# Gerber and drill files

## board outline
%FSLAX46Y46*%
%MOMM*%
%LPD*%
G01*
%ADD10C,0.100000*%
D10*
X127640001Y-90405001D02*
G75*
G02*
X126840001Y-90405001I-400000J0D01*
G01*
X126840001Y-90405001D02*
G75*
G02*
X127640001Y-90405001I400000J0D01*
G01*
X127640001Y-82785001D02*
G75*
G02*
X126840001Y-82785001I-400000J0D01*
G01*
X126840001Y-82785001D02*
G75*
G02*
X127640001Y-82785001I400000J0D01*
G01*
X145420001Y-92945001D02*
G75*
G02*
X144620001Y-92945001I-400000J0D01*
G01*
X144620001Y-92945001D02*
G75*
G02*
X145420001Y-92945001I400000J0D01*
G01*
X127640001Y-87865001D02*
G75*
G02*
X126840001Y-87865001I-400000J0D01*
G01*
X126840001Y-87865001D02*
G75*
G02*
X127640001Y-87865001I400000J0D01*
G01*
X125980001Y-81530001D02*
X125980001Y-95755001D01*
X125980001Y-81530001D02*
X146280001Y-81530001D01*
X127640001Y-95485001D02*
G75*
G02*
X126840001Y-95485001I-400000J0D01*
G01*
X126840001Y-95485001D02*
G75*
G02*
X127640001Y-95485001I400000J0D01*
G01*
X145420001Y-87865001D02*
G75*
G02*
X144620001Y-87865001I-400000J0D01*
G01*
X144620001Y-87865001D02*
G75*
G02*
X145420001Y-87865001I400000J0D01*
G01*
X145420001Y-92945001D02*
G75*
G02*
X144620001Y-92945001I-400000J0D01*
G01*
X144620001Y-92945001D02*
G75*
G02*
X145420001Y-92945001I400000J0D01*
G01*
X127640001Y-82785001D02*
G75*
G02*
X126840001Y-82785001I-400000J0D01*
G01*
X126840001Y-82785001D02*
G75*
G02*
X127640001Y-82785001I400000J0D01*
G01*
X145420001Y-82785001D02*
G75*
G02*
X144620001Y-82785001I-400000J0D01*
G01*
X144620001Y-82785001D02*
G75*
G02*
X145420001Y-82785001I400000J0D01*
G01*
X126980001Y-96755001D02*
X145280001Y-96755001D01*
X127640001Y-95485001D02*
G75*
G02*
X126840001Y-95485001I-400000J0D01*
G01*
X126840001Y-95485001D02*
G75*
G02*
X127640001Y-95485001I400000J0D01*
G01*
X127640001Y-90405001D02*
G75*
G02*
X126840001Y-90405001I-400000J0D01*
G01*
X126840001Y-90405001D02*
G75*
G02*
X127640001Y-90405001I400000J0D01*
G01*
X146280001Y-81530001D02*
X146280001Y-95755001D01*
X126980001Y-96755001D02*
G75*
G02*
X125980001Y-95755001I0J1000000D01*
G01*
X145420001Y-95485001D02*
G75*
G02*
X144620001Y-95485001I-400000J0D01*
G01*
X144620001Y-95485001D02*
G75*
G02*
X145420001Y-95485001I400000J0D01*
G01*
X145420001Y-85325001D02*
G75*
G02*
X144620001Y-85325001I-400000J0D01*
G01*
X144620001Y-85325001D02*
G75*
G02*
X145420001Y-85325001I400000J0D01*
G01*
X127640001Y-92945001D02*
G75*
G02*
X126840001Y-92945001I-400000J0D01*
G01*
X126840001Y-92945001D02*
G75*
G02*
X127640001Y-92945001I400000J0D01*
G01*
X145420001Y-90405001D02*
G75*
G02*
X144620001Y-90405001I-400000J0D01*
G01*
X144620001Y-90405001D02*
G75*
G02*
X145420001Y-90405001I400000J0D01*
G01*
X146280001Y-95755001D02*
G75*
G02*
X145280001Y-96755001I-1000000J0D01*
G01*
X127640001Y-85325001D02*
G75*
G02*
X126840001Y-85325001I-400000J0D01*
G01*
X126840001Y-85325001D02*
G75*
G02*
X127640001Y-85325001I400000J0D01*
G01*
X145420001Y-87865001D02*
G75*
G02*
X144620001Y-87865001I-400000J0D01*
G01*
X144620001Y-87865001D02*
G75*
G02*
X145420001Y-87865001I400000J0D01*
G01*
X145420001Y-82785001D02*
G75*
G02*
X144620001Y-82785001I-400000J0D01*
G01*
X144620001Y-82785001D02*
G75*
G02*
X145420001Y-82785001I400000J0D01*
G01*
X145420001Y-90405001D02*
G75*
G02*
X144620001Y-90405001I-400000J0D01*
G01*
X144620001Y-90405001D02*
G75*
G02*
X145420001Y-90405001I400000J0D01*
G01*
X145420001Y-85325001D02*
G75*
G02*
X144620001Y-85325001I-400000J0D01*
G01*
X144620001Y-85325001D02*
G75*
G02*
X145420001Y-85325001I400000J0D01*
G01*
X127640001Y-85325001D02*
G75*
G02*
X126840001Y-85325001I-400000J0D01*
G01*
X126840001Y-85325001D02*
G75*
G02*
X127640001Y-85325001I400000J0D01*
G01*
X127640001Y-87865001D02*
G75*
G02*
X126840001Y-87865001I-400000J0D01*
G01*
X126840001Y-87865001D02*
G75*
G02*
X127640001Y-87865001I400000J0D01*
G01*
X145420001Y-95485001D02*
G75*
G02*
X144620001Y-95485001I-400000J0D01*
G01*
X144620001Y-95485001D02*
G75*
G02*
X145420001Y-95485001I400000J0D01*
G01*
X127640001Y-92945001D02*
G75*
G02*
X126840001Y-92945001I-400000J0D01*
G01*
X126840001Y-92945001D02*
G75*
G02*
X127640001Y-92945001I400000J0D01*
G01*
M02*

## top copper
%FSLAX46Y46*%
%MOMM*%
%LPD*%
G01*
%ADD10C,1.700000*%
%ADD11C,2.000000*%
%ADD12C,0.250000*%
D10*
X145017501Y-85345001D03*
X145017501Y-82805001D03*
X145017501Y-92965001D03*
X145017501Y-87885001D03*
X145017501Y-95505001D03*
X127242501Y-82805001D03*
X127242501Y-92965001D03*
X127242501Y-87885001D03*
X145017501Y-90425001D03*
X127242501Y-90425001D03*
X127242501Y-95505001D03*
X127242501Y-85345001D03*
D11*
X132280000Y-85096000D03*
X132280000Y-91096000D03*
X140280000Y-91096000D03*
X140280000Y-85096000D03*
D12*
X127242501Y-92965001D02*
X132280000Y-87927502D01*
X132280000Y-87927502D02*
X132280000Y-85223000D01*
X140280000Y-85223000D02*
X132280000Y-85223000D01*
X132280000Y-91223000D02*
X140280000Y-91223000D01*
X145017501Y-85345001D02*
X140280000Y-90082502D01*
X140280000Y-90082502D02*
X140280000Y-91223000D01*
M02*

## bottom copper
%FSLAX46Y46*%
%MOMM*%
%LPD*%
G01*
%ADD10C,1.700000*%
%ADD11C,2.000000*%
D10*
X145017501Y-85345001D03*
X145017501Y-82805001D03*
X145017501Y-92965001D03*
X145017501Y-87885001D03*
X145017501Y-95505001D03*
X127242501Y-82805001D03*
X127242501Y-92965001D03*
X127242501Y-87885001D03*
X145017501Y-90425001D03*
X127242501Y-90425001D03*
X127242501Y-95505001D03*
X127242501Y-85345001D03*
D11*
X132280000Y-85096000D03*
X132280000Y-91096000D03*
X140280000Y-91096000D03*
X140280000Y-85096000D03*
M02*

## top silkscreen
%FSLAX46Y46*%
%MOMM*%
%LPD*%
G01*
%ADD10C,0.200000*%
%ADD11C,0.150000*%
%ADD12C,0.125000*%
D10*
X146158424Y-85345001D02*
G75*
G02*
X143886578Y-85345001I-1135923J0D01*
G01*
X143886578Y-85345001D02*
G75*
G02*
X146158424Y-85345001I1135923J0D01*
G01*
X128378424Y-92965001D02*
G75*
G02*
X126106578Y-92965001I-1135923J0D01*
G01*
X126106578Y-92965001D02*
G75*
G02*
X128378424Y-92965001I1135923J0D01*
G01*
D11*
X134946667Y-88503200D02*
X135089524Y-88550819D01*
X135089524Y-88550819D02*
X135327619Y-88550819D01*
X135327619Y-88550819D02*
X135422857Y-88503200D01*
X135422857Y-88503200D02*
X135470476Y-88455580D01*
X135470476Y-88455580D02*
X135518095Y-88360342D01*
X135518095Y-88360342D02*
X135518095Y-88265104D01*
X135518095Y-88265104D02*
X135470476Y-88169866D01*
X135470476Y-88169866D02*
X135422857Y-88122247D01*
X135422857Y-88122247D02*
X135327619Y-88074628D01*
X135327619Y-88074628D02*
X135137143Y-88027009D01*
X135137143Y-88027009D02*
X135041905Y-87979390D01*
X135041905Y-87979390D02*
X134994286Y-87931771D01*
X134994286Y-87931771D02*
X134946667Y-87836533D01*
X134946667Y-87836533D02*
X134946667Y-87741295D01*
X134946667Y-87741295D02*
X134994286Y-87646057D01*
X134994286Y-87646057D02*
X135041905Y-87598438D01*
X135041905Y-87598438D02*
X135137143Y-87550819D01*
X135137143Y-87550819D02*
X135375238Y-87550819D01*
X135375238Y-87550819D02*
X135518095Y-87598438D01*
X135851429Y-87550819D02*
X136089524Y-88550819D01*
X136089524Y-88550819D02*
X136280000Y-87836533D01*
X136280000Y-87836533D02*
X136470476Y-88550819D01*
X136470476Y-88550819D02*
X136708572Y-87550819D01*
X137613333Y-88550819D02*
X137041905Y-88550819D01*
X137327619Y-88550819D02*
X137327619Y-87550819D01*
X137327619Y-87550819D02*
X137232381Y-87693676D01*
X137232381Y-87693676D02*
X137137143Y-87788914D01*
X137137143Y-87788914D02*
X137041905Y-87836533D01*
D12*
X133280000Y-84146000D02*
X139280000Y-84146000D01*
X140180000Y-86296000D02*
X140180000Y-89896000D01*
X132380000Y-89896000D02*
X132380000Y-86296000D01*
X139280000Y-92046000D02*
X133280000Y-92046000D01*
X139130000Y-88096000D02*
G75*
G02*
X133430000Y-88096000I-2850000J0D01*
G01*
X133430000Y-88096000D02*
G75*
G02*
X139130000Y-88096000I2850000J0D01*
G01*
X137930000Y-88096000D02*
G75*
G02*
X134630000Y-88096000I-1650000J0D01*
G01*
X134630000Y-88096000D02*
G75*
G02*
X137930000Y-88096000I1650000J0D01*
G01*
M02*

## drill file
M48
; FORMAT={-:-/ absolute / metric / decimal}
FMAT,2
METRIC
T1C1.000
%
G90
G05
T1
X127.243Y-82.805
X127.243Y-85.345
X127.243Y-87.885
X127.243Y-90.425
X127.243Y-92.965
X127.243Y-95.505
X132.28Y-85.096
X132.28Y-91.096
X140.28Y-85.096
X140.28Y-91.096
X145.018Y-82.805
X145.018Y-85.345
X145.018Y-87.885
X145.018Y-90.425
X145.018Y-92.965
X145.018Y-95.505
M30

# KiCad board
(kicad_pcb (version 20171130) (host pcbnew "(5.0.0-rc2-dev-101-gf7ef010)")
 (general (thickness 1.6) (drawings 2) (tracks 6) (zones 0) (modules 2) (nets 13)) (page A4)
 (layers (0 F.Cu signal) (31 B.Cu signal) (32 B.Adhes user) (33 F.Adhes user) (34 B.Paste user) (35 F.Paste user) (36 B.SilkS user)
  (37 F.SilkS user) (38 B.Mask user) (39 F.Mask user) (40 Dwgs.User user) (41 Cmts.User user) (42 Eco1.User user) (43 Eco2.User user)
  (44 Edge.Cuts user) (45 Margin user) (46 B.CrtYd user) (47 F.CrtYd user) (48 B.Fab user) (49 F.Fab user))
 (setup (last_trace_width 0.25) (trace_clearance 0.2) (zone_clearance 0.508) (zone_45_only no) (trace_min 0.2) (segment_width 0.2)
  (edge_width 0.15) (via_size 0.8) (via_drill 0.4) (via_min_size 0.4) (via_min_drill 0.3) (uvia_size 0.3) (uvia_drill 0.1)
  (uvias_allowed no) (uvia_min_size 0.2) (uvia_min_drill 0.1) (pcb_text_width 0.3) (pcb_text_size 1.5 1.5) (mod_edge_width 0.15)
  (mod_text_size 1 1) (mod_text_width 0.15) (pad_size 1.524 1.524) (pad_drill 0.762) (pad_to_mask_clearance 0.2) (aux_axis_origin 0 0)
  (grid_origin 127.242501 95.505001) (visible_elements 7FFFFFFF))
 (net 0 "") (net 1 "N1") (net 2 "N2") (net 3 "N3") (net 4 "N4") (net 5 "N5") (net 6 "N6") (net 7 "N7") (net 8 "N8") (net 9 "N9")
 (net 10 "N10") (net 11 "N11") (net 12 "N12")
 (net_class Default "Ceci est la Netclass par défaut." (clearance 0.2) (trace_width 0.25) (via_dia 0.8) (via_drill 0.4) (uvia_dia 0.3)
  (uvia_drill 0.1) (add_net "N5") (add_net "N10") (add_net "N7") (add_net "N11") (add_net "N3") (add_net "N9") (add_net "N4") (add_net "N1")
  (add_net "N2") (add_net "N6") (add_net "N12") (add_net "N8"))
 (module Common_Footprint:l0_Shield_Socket (layer F.Cu) (at 136.130001 89.155001)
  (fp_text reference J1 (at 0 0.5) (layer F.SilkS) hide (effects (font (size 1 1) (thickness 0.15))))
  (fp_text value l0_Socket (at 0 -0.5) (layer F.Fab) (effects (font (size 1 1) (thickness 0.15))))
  (fp_circle (center -8.89 1.25) (end -8.49 1.25) (layer Edge.Cuts) (width 0.1))
  (fp_circle (center -8.89 -6.37) (end -8.49 -6.37) (layer Edge.Cuts) (width 0.1))
  (fp_circle (center 8.89 3.79) (end 9.29 3.79) (layer Edge.Cuts) (width 0.1))
  (fp_circle (center -8.89 -1.29) (end -8.49 -1.29) (layer Edge.Cuts) (width 0.1))
  (fp_line (start -10.15 -7.625) (end -10.15 6.6) (layer Edge.Cuts) (width 0.1))
  (fp_line (start -10.15 -7.625) (end 10.15 -7.625) (layer Edge.Cuts) (width 0.1))
  (fp_circle (center -8.89 6.33) (end -8.49 6.33) (layer Edge.Cuts) (width 0.1))
  (fp_circle (center 8.89 -1.29) (end 9.29 -1.29) (layer Edge.Cuts) (width 0.1))
  (fp_circle (center 8.89 3.79) (end 9.29 3.79) (layer Edge.Cuts) (width 0.1))
  (fp_circle (center -8.89 -6.37) (end -8.49 -6.37) (layer Edge.Cuts) (width 0.1))
  (fp_circle (center 8.89 -6.37) (end 9.29 -6.37) (layer Edge.Cuts) (width 0.1))
  (fp_line (start -9.15 7.6) (end 9.15 7.6) (layer Edge.Cuts) (width 0.1))
  (fp_circle (center -8.89 6.33) (end -8.49 6.33) (layer Edge.Cuts) (width 0.1))
  (fp_circle (center -8.89 1.25) (end -8.49 1.25) (layer Edge.Cuts) (width 0.1))
  (fp_line (start 10.15 -7.625) (end 10.15 6.6) (layer Edge.Cuts) (width 0.1))
  (fp_arc (start -9.15 6.6) (end -10.15 6.6) (angle -90) (layer Edge.Cuts) (width 0.1))
  (fp_circle (center 8.89 6.33) (end 9.29 6.33) (layer Edge.Cuts) (width 0.1))
  (fp_circle (center 8.89 -3.83) (end 9.29 -3.83) (layer Edge.Cuts) (width 0.1))
  (fp_circle (center -8.89 3.79) (end -8.49 3.79) (layer Edge.Cuts) (width 0.1))
  (fp_circle (center 8.89 1.25) (end 9.29 1.25) (layer Edge.Cuts) (width 0.1))
  (fp_arc (start 9.15 6.6) (end 9.15 7.6) (angle -90) (layer Edge.Cuts) (width 0.1))
  (fp_circle (center -8.89 -3.83) (end -8.49 -3.83) (layer Edge.Cuts) (width 0.1))
  (fp_circle (center 8.89 -1.29) (end 9.29 -1.29) (layer Edge.Cuts) (width 0.1))
  (fp_circle (center 8.89 -6.37) (end 9.29 -6.37) (layer Edge.Cuts) (width 0.1))
  (fp_circle (center 8.89 1.25) (end 9.29 1.25) (layer Edge.Cuts) (width 0.1))
  (fp_circle (center 8.89 -3.83) (end 9.29 -3.83) (layer Edge.Cuts) (width 0.1))
  (fp_circle (center -8.89 -3.83) (end -8.49 -3.83) (layer Edge.Cuts) (width 0.1))
  (fp_circle (center -8.89 -1.29) (end -8.49 -1.29) (layer Edge.Cuts) (width 0.1))
  (fp_circle (center 8.89 6.33) (end 9.29 6.33) (layer Edge.Cuts) (width 0.1))
  (fp_circle (center -8.89 3.79) (end -8.49 3.79) (layer Edge.Cuts) (width 0.1))
  (pad 5 thru_hole circle (at 8.8875 -3.81 270) (size 1.7 1.7) (drill 1) (layers *.Cu *.Mask) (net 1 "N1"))
  (pad 6 thru_hole circle (at 8.8875 -6.35 270) (size 1.7 1.7) (drill 1) (layers *.Cu *.Mask) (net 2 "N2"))
  (pad 2 thru_hole circle (at 8.8875 3.81 270) (size 1.7 1.7) (drill 1) (layers *.Cu *.Mask) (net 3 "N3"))
  (pad 4 thru_hole circle (at 8.8875 -1.27 270) (size 1.7 1.7) (drill 1) (layers *.Cu *.Mask) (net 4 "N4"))
  (pad 1 thru_hole circle (at 8.8875 6.35 270) (size 1.7 1.7) (drill 1) (layers *.Cu *.Mask) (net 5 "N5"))
  (pad 7 thru_hole circle (at -8.8875 -6.35 270) (size 1.7 1.7) (drill 1) (layers *.Cu *.Mask) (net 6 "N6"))
  (pad 11 thru_hole circle (at -8.8875 3.81 270) (size 1.7 1.7) (drill 1) (layers *.Cu *.Mask) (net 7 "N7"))
  (pad 9 thru_hole circle (at -8.8875 -1.27 270) (size 1.7 1.7) (drill 1) (layers *.Cu *.Mask) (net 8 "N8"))
  (pad 3 thru_hole circle (at 8.8875 1.27 270) (size 1.7 1.7) (drill 1) (layers *.Cu *.Mask) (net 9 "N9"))
  (pad 10 thru_hole circle (at -8.8875 1.27 270) (size 1.7 1.7) (drill 1) (layers *.Cu *.Mask) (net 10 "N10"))
  (pad 12 thru_hole circle (at -8.8875 6.35 270) (size 1.7 1.7) (drill 1) (layers *.Cu *.Mask) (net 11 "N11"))
  (pad 8 thru_hole circle (at -8.8875 -3.81 270) (size 1.7 1.7) (drill 1) (layers *.Cu *.Mask) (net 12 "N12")))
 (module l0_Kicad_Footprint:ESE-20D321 (layer F.Cu) (at 136.28 88.096)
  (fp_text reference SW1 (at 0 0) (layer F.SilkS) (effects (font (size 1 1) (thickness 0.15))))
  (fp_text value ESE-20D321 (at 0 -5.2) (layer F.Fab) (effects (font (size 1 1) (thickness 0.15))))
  (fp_line (start -3 -3.95) (end 3 -3.95) (layer F.SilkS) (width 0.125))
  (fp_line (start 3.9 -1.8) (end 3.9 1.8) (layer F.SilkS) (width 0.125))
  (fp_line (start -3.9 1.8) (end -3.9 -1.8) (layer F.SilkS) (width 0.125))
  (fp_line (start 3 3.95) (end -3 3.95) (layer F.SilkS) (width 0.125))
  (fp_circle (center 0 0) (end 2.85 0) (layer F.SilkS) (width 0.125))
  (fp_circle (center 0 0) (end 1.65 0) (layer F.SilkS) (width 0.125))
  (pad 1 thru_hole circle (at -4 -3) (size 2 2) (drill 1) (layers *.Cu *.Mask) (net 7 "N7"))
  (pad 2 thru_hole circle (at -4 3) (size 2 2) (drill 1) (layers *.Cu *.Mask) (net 1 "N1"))
  (pad 2 thru_hole circle (at 4 3) (size 2 2) (drill 1) (layers *.Cu *.Mask) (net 1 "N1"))
  (pad 1 thru_hole circle (at 4 -3) (size 2 2) (drill 1) (layers *.Cu *.Mask) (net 7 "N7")))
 (gr_circle (center 145.022501 85.345001) (end 146.038501 85.853001) (layer F.SilkS) (width 0.2))
 (gr_circle (center 127.242501 92.965001) (end 128.258501 93.473001) (layer F.SilkS) (width 0.2))
 (segment (start 127.242501 92.965001) (end 132.28 87.927502) (width 0.25) (layer F.Cu) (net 7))
 (segment (start 132.28 87.927502) (end 132.28 85.223) (width 0.25) (layer F.Cu) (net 7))
 (segment (start 140.28 85.223) (end 132.28 85.223) (width 0.25) (layer F.Cu) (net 7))
 (segment (start 132.28 91.223) (end 140.28 91.223) (width 0.25) (layer F.Cu) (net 1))
 (segment (start 145.017501 85.345001) (end 140.28 90.082502) (width 0.25) (layer F.Cu) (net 1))
 (segment (start 140.28 90.082502) (end 140.28 91.223) (width 0.25) (layer F.Cu) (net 1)))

